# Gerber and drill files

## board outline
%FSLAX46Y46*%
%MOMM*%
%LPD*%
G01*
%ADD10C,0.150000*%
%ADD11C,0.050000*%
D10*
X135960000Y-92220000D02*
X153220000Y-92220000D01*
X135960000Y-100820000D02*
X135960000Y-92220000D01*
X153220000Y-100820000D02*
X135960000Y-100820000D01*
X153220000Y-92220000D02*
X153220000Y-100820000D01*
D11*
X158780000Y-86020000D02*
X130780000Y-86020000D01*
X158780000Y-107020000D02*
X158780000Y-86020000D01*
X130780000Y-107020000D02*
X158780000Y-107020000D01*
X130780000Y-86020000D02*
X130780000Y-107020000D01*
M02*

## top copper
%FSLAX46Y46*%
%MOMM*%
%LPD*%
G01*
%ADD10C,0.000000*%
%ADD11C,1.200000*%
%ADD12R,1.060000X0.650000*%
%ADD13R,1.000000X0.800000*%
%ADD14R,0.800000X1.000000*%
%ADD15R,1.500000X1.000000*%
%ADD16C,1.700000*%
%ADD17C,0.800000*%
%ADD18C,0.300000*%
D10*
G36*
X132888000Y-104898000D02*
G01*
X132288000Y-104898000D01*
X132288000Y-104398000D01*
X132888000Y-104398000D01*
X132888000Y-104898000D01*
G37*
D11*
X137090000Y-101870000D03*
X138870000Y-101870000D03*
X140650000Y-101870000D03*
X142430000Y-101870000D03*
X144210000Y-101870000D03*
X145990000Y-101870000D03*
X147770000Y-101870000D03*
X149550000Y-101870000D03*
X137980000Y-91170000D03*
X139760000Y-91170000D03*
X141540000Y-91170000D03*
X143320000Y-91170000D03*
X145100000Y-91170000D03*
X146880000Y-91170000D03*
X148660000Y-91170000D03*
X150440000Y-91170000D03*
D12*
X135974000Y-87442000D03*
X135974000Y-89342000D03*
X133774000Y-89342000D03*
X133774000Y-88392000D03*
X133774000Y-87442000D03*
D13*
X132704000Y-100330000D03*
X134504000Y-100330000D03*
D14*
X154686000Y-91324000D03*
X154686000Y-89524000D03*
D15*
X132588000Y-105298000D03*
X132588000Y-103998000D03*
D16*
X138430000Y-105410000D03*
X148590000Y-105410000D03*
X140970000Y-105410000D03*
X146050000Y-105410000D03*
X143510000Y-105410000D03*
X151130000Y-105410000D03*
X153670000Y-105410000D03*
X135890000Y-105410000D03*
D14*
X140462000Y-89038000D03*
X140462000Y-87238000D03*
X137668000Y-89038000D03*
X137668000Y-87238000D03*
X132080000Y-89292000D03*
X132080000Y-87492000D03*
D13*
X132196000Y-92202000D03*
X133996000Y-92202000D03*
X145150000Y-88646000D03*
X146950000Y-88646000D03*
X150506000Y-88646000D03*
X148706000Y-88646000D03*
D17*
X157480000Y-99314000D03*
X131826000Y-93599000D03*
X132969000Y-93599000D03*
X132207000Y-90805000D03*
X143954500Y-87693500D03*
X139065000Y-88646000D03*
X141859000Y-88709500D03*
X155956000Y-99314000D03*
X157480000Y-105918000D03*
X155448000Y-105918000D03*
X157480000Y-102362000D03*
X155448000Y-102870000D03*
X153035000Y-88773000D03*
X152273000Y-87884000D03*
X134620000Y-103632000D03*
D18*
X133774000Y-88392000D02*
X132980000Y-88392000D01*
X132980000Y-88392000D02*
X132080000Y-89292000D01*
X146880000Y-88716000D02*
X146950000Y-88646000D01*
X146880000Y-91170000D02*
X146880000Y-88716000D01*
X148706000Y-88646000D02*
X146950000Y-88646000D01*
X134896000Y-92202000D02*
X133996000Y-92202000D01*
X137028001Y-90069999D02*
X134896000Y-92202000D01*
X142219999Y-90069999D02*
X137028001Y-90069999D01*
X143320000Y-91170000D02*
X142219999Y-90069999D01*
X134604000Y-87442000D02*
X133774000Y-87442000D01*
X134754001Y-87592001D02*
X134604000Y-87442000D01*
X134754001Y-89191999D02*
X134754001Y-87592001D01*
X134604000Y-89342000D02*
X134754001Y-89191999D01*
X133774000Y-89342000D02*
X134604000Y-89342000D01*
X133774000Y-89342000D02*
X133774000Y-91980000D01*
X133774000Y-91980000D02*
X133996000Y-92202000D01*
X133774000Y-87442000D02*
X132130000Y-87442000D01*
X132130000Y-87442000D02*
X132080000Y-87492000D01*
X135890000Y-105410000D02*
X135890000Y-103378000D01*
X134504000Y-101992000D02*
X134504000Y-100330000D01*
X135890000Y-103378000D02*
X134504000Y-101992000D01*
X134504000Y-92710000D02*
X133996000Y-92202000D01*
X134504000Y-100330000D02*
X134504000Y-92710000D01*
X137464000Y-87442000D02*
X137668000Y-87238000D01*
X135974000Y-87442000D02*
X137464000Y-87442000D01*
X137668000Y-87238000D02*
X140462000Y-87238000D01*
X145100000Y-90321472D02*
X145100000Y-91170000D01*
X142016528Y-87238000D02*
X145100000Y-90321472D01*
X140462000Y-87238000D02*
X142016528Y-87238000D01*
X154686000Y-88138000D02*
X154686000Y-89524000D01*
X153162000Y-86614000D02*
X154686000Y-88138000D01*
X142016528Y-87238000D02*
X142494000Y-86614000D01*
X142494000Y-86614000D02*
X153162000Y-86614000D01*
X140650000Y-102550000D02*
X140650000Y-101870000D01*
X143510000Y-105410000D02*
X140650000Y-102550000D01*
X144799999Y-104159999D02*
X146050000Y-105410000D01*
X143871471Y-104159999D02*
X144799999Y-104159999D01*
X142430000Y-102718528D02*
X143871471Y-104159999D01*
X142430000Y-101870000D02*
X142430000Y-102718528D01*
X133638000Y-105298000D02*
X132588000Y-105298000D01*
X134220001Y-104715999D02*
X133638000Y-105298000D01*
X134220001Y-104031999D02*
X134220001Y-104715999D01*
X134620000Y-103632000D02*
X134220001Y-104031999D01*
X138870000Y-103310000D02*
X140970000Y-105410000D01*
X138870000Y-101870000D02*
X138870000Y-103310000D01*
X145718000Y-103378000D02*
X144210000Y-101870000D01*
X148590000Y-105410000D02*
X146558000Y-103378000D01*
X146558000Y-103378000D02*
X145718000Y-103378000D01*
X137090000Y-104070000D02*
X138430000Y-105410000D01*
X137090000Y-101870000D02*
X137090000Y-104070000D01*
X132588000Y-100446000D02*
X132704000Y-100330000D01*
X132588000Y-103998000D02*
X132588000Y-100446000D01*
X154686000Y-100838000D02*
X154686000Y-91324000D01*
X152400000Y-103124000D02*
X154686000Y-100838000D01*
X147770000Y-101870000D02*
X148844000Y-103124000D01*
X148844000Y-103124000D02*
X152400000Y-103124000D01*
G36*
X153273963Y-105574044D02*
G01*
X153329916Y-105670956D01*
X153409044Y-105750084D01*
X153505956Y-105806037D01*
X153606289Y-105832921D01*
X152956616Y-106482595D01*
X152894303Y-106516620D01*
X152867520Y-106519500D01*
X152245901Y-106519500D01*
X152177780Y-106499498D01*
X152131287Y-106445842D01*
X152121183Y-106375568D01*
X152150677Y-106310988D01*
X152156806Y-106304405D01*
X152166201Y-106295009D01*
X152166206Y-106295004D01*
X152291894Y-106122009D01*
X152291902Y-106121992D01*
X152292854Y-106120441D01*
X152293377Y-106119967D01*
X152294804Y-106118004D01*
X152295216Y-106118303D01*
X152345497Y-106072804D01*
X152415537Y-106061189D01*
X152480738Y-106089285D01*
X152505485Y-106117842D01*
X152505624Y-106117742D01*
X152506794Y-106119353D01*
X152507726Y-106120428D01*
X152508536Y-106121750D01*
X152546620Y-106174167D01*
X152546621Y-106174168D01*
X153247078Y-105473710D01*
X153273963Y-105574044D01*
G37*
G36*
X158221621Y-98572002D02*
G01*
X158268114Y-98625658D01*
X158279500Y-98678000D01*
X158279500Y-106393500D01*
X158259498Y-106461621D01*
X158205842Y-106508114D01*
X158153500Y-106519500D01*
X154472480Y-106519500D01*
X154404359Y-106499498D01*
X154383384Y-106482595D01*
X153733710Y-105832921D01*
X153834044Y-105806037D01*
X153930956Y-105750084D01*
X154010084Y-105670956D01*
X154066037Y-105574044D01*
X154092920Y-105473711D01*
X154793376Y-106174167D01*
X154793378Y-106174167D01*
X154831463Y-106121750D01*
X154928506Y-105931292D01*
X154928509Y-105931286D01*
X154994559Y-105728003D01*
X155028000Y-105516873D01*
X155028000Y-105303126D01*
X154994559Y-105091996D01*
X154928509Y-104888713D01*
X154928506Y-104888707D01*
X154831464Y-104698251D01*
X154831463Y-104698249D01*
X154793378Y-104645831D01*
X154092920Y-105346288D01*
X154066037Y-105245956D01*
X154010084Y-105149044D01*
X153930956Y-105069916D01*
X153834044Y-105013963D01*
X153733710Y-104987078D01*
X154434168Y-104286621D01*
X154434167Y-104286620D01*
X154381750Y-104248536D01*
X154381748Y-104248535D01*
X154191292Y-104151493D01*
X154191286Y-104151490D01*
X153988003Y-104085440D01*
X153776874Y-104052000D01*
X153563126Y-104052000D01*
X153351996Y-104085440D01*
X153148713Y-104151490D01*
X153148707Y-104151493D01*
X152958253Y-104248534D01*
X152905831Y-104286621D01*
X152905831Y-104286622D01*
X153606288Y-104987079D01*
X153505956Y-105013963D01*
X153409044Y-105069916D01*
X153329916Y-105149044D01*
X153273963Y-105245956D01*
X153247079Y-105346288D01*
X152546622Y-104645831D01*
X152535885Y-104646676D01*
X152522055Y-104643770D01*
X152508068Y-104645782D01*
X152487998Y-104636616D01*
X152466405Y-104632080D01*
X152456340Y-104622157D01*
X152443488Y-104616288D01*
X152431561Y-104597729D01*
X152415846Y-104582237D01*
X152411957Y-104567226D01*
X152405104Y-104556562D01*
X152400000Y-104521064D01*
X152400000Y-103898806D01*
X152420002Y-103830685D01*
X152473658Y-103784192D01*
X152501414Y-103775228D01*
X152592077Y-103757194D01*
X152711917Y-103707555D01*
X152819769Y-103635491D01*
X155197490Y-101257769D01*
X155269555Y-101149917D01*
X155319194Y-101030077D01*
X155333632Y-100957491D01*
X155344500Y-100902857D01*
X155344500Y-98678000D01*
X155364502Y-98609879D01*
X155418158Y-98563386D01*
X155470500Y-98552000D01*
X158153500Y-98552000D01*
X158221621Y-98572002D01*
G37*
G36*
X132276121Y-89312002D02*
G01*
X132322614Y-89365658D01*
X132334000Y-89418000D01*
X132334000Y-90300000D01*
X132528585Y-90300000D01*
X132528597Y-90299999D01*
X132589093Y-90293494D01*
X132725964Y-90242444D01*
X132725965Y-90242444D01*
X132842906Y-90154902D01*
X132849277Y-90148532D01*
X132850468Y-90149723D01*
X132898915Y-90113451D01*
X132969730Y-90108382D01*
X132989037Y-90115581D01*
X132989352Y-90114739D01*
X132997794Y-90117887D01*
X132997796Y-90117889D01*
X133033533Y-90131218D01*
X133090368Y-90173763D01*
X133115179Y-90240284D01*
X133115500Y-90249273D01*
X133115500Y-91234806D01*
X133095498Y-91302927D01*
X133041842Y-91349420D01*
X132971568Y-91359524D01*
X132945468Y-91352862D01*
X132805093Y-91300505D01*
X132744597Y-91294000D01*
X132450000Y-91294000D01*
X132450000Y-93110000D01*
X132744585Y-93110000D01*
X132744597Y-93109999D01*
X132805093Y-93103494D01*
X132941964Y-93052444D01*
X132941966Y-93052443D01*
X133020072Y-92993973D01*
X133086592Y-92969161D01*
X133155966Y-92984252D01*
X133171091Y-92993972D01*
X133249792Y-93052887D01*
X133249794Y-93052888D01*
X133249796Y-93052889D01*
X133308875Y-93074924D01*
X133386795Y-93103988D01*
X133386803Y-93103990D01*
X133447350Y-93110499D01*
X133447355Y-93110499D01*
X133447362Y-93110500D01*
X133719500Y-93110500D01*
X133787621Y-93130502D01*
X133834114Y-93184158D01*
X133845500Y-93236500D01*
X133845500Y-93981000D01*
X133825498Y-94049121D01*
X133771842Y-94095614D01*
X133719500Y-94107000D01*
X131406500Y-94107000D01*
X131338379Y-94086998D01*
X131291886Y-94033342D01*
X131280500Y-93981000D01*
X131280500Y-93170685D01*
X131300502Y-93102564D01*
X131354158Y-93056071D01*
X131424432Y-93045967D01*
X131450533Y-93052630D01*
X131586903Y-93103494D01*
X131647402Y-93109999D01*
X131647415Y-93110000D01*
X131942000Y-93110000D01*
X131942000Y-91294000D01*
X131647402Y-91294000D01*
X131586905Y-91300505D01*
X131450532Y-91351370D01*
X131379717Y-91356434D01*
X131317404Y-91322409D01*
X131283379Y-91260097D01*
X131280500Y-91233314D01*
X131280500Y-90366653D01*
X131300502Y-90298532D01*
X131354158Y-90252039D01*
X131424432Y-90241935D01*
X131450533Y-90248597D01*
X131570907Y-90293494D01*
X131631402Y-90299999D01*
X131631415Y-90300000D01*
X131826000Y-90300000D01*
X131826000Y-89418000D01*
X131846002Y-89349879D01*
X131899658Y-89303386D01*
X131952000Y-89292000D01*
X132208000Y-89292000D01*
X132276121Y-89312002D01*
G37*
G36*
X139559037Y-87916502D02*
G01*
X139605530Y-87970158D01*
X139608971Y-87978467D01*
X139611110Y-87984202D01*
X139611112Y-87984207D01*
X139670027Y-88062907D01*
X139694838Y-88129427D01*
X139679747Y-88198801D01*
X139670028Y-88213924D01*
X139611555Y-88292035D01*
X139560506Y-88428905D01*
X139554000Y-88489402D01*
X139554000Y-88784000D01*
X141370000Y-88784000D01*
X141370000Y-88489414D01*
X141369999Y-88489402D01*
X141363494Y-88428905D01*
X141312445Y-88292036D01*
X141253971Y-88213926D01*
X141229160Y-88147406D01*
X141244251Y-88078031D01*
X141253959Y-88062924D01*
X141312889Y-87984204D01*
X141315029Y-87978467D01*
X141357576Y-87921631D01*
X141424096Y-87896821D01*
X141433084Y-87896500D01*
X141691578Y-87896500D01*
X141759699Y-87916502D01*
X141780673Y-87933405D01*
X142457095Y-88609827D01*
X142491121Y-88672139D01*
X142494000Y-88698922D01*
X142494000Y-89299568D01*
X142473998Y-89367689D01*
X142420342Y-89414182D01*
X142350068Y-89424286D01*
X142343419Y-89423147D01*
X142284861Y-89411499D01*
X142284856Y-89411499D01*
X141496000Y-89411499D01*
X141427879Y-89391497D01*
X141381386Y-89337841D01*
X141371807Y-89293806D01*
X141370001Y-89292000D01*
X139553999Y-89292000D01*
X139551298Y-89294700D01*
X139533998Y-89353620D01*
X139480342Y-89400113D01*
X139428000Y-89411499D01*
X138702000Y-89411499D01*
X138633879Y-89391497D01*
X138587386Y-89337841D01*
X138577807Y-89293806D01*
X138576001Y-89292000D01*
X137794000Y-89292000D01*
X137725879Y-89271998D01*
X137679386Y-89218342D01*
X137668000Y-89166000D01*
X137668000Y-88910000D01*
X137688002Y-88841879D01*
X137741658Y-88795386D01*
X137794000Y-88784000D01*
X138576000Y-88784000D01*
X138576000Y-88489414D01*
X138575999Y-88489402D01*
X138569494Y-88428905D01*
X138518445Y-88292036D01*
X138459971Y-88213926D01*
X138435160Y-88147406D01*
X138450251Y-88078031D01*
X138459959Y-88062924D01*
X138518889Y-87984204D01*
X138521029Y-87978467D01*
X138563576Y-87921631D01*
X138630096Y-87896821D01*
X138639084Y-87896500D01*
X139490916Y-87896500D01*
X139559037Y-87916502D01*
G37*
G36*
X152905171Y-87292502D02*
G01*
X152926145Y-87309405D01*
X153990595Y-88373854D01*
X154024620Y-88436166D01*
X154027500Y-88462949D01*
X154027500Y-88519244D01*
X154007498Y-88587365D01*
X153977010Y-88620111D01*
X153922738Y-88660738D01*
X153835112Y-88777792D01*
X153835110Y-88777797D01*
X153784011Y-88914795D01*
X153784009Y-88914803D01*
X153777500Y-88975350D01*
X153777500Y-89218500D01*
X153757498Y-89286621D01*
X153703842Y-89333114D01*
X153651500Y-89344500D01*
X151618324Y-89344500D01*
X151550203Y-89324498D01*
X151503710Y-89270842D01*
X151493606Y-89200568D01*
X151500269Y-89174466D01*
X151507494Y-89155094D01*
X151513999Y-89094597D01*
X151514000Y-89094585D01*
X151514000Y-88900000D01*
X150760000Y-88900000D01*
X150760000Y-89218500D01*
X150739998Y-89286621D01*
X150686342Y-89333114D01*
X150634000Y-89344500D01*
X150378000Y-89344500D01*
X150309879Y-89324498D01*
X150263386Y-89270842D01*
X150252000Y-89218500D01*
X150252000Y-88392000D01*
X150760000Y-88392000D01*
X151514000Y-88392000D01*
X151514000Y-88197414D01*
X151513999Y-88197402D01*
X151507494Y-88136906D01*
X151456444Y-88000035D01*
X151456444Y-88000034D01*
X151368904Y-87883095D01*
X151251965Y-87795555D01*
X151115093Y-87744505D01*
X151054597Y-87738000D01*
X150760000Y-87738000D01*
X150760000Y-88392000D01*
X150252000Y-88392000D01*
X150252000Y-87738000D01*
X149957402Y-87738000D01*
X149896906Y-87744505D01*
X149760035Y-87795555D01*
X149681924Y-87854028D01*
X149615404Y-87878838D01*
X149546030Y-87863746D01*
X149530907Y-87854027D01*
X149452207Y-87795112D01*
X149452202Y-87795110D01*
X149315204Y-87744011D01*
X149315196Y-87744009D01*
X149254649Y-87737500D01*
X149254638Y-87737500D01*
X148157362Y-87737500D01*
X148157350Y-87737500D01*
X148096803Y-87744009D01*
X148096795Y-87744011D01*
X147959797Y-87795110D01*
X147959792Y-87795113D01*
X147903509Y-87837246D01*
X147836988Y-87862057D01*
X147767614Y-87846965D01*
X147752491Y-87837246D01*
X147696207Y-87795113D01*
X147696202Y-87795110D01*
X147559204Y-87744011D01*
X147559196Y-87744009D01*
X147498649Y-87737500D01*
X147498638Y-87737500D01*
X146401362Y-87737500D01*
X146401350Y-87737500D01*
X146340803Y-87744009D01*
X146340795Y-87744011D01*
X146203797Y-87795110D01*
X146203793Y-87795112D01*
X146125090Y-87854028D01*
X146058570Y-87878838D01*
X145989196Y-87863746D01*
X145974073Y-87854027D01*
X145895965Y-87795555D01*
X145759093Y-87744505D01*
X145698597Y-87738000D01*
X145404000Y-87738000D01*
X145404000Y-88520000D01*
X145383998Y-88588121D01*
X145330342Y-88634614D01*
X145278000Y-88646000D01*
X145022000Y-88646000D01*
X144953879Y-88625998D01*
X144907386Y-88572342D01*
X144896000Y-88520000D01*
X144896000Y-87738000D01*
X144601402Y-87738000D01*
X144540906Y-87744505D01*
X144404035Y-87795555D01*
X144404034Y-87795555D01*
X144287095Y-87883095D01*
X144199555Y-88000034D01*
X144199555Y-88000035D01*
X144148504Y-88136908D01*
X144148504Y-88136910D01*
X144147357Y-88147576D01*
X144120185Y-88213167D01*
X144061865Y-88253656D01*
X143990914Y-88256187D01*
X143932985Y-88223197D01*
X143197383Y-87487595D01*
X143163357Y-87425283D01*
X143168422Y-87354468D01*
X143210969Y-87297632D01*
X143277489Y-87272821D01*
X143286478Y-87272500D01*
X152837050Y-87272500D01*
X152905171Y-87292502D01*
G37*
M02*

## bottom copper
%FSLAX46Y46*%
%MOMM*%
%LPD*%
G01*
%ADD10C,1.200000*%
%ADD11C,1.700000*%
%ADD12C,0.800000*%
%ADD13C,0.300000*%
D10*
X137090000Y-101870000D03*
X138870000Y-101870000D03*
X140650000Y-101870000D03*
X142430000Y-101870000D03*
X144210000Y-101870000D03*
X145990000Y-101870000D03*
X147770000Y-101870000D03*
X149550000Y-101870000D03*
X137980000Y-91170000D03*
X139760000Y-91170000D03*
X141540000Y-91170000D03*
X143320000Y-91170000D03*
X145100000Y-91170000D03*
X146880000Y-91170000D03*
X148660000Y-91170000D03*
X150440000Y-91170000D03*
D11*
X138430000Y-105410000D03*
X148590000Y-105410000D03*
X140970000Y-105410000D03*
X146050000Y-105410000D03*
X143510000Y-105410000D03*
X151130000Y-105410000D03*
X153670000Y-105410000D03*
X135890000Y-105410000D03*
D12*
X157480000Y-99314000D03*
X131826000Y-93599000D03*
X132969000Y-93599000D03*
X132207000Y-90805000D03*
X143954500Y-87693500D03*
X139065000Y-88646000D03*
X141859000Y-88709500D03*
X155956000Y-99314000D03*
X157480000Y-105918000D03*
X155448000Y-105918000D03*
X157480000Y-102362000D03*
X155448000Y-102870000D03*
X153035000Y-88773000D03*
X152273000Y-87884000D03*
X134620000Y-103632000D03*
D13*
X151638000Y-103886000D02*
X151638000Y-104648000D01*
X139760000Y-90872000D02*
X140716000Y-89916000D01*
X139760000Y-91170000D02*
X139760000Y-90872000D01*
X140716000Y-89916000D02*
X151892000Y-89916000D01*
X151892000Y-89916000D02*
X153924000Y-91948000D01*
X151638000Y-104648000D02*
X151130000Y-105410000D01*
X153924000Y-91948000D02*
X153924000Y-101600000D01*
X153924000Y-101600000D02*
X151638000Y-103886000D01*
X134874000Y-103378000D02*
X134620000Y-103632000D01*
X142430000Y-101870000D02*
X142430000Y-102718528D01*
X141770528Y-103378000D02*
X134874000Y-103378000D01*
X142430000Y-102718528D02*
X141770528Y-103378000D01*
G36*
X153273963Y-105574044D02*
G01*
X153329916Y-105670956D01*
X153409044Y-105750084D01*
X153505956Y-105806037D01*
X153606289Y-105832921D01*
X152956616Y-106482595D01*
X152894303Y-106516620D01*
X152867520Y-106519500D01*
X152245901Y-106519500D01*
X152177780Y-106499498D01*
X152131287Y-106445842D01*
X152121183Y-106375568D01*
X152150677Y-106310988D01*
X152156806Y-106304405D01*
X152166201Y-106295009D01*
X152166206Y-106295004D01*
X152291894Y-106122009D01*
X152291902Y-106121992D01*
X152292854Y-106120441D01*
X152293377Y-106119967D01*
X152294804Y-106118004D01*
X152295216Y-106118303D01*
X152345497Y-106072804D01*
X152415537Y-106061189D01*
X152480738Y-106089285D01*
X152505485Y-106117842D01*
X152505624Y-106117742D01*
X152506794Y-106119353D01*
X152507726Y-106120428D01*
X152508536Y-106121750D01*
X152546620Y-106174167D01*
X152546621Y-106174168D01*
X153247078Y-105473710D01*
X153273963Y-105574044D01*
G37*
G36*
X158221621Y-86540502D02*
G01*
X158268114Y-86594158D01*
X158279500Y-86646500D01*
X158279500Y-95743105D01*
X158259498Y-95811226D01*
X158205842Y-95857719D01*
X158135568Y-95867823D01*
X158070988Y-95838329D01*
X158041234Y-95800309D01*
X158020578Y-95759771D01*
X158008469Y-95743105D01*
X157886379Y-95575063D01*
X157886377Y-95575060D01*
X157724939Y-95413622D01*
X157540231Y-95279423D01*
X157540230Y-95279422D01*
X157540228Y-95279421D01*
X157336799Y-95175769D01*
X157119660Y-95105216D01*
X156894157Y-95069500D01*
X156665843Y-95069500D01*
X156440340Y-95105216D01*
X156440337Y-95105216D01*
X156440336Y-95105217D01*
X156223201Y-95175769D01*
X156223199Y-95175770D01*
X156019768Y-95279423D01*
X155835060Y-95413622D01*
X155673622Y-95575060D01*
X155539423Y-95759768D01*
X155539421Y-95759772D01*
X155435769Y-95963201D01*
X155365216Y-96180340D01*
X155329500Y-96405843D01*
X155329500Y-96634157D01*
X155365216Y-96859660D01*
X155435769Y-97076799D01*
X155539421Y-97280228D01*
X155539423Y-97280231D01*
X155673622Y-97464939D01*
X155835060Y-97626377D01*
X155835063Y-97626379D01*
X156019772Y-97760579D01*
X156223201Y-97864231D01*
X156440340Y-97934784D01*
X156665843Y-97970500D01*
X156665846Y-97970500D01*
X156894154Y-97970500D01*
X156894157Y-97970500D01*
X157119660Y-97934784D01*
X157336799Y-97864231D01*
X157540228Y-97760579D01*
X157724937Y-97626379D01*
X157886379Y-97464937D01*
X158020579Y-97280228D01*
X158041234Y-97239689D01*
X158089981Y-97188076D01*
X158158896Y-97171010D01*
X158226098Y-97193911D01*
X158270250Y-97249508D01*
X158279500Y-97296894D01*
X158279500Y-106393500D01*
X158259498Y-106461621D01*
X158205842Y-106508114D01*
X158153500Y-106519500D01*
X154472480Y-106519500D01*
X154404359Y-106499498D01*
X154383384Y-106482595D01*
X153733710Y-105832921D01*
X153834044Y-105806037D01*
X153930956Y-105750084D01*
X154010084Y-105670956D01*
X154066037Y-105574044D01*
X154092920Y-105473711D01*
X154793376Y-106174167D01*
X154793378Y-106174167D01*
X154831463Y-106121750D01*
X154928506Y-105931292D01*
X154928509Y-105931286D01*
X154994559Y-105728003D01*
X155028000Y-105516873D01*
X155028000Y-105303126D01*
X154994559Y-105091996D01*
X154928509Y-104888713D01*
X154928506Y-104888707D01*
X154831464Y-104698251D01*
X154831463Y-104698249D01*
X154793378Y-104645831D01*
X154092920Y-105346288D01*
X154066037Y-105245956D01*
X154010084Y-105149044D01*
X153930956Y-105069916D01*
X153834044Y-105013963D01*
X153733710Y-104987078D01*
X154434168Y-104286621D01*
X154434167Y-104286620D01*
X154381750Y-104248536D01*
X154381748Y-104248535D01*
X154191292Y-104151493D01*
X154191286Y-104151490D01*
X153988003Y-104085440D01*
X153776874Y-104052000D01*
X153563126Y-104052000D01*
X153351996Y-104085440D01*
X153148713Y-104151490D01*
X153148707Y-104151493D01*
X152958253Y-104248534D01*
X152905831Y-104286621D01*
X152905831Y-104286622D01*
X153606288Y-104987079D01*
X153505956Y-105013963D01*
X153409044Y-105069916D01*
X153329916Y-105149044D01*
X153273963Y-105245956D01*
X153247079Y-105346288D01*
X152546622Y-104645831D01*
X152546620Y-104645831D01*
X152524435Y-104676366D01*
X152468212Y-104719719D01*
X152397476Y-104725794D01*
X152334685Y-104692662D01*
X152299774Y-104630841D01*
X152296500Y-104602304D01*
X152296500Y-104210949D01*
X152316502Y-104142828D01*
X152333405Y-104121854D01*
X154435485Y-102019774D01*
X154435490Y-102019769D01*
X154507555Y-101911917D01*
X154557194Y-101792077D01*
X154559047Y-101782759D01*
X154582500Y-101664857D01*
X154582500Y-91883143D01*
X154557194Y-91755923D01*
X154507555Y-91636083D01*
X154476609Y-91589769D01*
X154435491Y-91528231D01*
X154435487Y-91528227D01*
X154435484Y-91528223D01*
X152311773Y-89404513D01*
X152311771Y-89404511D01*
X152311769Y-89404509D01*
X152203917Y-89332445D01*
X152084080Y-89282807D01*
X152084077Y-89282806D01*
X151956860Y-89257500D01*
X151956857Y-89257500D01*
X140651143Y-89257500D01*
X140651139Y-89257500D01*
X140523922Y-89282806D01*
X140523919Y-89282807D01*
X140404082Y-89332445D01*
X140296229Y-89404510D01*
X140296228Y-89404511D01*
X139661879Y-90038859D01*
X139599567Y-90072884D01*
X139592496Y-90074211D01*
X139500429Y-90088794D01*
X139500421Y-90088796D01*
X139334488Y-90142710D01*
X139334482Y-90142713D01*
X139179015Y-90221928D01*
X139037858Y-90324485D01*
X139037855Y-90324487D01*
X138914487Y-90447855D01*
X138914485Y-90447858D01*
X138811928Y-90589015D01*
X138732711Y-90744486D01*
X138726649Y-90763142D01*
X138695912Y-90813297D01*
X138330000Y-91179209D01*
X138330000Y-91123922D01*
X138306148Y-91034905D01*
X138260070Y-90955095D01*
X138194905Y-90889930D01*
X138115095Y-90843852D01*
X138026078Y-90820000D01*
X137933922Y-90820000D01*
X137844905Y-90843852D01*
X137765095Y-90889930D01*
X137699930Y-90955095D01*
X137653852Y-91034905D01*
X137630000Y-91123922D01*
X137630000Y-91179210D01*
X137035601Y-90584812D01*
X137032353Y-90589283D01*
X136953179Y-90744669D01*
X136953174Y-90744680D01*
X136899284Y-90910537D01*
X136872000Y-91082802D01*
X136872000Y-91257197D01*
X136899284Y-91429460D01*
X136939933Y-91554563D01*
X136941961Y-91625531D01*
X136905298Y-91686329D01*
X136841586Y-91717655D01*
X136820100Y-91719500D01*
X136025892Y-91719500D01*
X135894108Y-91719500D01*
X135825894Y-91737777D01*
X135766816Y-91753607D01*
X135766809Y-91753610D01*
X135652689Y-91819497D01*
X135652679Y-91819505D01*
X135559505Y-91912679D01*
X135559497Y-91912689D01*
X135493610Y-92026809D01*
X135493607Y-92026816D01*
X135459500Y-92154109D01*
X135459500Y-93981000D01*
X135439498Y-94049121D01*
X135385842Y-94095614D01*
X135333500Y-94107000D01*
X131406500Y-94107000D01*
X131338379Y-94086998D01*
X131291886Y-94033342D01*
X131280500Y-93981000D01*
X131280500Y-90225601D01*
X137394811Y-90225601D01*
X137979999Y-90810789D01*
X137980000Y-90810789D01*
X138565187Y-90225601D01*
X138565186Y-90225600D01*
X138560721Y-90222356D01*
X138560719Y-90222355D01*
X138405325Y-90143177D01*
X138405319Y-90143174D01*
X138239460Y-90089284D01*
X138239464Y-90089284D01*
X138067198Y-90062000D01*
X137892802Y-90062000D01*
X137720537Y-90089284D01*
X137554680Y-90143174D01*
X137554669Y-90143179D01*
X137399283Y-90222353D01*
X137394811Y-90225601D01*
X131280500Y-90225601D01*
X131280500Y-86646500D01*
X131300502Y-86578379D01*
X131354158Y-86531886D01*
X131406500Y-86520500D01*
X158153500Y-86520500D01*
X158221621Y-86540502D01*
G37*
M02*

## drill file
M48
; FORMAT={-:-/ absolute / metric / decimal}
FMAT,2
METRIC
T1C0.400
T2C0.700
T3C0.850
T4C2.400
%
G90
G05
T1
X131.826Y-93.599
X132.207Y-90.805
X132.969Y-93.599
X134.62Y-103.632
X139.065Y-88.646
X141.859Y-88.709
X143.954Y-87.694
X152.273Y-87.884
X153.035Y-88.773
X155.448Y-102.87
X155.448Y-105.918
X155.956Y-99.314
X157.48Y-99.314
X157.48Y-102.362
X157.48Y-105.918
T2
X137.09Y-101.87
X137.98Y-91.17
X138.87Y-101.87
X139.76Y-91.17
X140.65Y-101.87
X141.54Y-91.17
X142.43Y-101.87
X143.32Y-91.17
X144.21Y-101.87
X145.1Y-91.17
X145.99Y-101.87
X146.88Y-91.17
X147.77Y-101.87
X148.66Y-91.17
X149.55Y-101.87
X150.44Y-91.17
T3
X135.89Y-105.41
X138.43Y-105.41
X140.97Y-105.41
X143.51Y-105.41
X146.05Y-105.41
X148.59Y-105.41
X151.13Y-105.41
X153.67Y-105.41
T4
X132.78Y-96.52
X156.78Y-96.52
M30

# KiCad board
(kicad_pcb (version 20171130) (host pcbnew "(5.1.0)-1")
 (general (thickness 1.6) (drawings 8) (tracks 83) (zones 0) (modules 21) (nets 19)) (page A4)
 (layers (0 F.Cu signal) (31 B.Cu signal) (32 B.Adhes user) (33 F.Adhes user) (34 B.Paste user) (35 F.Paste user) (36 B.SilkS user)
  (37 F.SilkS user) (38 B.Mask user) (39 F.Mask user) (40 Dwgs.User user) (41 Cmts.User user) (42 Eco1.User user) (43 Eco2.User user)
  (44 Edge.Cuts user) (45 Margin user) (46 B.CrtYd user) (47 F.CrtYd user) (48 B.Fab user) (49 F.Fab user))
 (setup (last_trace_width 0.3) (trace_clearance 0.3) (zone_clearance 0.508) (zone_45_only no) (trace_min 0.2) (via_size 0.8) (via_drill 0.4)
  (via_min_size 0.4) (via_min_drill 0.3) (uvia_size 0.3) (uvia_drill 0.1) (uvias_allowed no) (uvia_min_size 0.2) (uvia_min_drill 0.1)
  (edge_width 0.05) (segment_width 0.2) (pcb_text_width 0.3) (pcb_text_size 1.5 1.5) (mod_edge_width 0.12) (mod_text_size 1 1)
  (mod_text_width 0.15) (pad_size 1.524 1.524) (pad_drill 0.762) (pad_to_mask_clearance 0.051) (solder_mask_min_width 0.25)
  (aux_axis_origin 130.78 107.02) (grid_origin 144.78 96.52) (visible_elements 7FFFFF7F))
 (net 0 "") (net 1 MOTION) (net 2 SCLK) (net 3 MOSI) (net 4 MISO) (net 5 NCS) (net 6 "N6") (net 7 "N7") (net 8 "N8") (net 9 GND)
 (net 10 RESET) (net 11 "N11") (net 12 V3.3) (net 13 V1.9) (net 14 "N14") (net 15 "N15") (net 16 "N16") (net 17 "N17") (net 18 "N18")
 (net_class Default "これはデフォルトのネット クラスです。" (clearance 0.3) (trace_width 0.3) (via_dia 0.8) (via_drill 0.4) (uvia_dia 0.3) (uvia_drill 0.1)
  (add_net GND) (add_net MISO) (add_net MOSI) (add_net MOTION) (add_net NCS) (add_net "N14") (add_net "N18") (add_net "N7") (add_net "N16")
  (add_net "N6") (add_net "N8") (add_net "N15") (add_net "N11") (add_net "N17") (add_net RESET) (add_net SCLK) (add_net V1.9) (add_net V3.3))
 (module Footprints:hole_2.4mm (layer F.Cu) (at 132.78 96.52)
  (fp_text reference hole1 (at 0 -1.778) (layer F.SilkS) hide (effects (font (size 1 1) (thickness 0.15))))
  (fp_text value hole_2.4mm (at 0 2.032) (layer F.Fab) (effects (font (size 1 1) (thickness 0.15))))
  (pad "" np_thru_hole circle (at 0 0) (size 2.4 2.4) (drill 2.4) (layers *.Cu *.Mask)))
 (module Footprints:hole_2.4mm (layer F.Cu) (at 156.78 96.52)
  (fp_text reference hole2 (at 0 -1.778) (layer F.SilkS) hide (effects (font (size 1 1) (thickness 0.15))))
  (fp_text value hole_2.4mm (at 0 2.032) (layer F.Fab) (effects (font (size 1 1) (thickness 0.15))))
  (pad "" np_thru_hole circle (at 0 0) (size 2.4 2.4) (drill 2.4) (layers *.Cu *.Mask)))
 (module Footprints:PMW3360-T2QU (layer F.Cu) (at 144.78 96.52)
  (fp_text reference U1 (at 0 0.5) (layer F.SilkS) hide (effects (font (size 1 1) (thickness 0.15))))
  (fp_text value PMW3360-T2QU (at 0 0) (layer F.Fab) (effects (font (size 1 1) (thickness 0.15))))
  (pad 9 thru_hole circle (at -7.69 5.35) (size 1.2 1.2) (drill 0.7) (layers *.Cu *.Mask) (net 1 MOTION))
  (pad 10 thru_hole circle (at -5.91 5.35) (size 1.2 1.2) (drill 0.7) (layers *.Cu *.Mask) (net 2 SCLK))
  (pad 11 thru_hole circle (at -4.13 5.35) (size 1.2 1.2) (drill 0.7) (layers *.Cu *.Mask) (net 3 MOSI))
  (pad 12 thru_hole circle (at -2.35 5.35) (size 1.2 1.2) (drill 0.7) (layers *.Cu *.Mask) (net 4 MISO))
  (pad 13 thru_hole circle (at -0.57 5.35) (size 1.2 1.2) (drill 0.7) (layers *.Cu *.Mask) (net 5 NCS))
  (pad 14 thru_hole circle (at 1.21 5.35) (size 1.2 1.2) (drill 0.7) (layers *.Cu *.Mask) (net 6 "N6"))
  (pad 15 thru_hole circle (at 2.99 5.35) (size 1.2 1.2) (drill 0.7) (layers *.Cu *.Mask) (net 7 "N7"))
  (pad 16 thru_hole circle (at 4.77 5.35) (size 1.2 1.2) (drill 0.7) (layers *.Cu *.Mask) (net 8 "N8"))
  (pad 8 thru_hole circle (at -6.8 -5.35) (size 1.2 1.2) (drill 0.7) (layers *.Cu *.Mask) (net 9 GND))
  (pad 7 thru_hole circle (at -5.02 -5.35) (size 1.2 1.2) (drill 0.7) (layers *.Cu *.Mask) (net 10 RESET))
  (pad 6 thru_hole circle (at -3.24 -5.35) (size 1.2 1.2) (drill 0.7) (layers *.Cu *.Mask) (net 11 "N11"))
  (pad 5 thru_hole circle (at -1.46 -5.35) (size 1.2 1.2) (drill 0.7) (layers *.Cu *.Mask) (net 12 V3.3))
  (pad 4 thru_hole circle (at 0.32 -5.35) (size 1.2 1.2) (drill 0.7) (layers *.Cu *.Mask) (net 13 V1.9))
  (pad 3 thru_hole circle (at 2.1 -5.35) (size 1.2 1.2) (drill 0.7) (layers *.Cu *.Mask) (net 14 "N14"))
  (pad 2 thru_hole circle (at 3.88 -5.35) (size 1.2 1.2) (drill 0.7) (layers *.Cu *.Mask) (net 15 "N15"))
  (pad 1 thru_hole circle (at 5.66 -5.35) (size 1.2 1.2) (drill 0.7) (layers *.Cu *.Mask) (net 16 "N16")))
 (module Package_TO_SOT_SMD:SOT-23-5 (layer F.Cu) (at 134.874 88.392)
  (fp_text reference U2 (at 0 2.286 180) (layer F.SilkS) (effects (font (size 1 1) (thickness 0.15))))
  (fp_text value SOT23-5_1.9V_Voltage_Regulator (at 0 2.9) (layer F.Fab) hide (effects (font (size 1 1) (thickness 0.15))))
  (pad 5 smd rect (at 1.1 -0.95) (size 1.06 0.65) (layers F.Cu F.Paste F.Mask) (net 13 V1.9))
  (pad 4 smd rect (at 1.1 0.95) (size 1.06 0.65) (layers F.Cu F.Paste F.Mask) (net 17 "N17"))
  (pad 3 smd rect (at -1.1 0.95) (size 1.06 0.65) (layers F.Cu F.Paste F.Mask) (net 12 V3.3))
  (pad 2 smd rect (at -1.1 0) (size 1.06 0.65) (layers F.Cu F.Paste F.Mask) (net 9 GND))
  (pad 1 smd rect (at -1.1 -0.95) (size 1.06 0.65) (layers F.Cu F.Paste F.Mask) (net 12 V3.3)))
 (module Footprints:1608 (layer F.Cu) (at 133.604 100.33 180)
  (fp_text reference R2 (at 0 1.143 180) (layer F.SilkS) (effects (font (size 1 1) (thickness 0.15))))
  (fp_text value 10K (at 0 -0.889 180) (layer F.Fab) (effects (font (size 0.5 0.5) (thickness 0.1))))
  (pad 2 smd rect (at 0.9 0 180) (size 1 0.8) (layers F.Cu F.Paste F.Mask) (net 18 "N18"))
  (pad 1 smd rect (at -0.9 0 180) (size 1 0.8) (layers F.Cu F.Paste F.Mask) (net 12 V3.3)))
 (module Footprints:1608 (layer F.Cu) (at 154.686 90.424 270)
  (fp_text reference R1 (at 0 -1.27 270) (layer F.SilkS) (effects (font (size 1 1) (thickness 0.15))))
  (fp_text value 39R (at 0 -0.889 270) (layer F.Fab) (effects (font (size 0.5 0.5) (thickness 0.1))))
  (pad 2 smd rect (at 0.9 0 270) (size 1 0.8) (layers F.Cu F.Paste F.Mask) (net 7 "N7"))
  (pad 1 smd rect (at -0.9 0 270) (size 1 0.8) (layers F.Cu F.Paste F.Mask) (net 13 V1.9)))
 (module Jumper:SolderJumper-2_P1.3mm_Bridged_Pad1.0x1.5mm (layer F.Cu) (at 132.588 104.648 270)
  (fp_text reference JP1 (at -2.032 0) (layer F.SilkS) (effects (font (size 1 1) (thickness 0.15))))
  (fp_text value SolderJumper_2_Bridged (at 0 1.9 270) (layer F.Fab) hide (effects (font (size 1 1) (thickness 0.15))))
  (fp_poly (pts (xy -0.25 -0.3) (xy 0.25 -0.3) (xy 0.25 0.3) (xy -0.25 0.3)) (layer F.Cu) (width 0))
  (pad 2 smd rect (at 0.65 0 270) (size 1 1.5) (layers F.Cu F.Mask) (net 4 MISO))
  (pad 1 smd rect (at -0.65 0 270) (size 1 1.5) (layers F.Cu F.Mask) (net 18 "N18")))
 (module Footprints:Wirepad (layer F.Cu) (at 138.43 105.41 180)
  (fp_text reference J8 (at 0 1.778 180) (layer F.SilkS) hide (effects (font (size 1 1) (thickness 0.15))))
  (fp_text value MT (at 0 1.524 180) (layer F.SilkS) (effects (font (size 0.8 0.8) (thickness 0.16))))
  (pad 1 thru_hole circle (at 0 0 180) (size 1.7 1.7) (drill 0.85) (layers *.Cu *.Mask) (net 1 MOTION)))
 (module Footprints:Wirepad (layer F.Cu) (at 148.59 105.41 180)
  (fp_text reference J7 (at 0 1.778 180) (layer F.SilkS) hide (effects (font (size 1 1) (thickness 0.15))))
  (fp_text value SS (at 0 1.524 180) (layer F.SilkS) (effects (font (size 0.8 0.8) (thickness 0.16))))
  (pad 1 thru_hole circle (at 0 0 180) (size 1.7 1.7) (drill 0.85) (layers *.Cu *.Mask) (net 5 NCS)))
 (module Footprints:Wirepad (layer F.Cu) (at 140.97 105.41 180)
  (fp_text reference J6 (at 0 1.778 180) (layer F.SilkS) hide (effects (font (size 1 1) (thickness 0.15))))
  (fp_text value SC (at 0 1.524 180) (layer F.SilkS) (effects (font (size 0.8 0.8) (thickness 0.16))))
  (pad 1 thru_hole circle (at 0 0 180) (size 1.7 1.7) (drill 0.85) (layers *.Cu *.Mask) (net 2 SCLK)))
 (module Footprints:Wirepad (layer F.Cu) (at 146.05 105.41 180)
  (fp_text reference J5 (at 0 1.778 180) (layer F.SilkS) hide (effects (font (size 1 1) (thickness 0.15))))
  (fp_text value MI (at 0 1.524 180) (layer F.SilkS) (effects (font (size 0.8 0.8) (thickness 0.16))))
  (pad 1 thru_hole circle (at 0 0 180) (size 1.7 1.7) (drill 0.85) (layers *.Cu *.Mask) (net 4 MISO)))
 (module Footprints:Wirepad (layer F.Cu) (at 143.51 105.41 180)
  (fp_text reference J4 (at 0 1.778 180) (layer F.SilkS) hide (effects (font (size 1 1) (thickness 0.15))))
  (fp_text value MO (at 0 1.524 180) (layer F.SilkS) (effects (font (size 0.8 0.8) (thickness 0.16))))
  (pad 1 thru_hole circle (at 0 0 180) (size 1.7 1.7) (drill 0.85) (layers *.Cu *.Mask) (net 3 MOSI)))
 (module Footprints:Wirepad (layer F.Cu) (at 151.13 105.41 180)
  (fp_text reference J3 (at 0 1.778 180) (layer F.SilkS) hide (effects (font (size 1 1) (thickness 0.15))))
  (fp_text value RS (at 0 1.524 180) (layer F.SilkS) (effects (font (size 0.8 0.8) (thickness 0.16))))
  (pad 1 thru_hole circle (at 0 0 180) (size 1.7 1.7) (drill 0.85) (layers *.Cu *.Mask) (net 10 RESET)))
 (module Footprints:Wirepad (layer F.Cu) (at 153.67 105.41 180)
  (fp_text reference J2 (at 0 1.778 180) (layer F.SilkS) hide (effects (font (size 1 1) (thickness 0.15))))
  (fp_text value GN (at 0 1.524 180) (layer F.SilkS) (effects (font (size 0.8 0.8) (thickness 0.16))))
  (pad 1 thru_hole circle (at 0 0 180) (size 1.7 1.7) (drill 0.85) (layers *.Cu *.Mask) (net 9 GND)))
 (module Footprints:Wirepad (layer F.Cu) (at 135.89 105.41 180)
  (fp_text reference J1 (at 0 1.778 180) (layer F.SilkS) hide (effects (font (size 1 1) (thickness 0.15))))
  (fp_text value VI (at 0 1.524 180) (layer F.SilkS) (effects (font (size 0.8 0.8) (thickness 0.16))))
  (pad 1 thru_hole circle (at 0 0 180) (size 1.7 1.7) (drill 0.85) (layers *.Cu *.Mask) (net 12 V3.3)))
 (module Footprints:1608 (layer F.Cu) (at 140.462 88.138 270)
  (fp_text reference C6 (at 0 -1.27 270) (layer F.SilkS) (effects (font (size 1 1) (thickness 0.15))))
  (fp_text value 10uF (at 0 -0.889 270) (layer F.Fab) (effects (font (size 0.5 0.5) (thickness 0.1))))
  (pad 2 smd rect (at 0.9 0 270) (size 1 0.8) (layers F.Cu F.Paste F.Mask) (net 9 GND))
  (pad 1 smd rect (at -0.9 0 270) (size 1 0.8) (layers F.Cu F.Paste F.Mask) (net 13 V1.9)))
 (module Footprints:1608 (layer F.Cu) (at 137.668 88.138 270)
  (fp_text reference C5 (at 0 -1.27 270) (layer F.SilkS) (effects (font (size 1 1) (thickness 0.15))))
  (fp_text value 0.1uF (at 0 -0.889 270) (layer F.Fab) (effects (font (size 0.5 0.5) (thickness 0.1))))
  (pad 2 smd rect (at 0.9 0 270) (size 1 0.8) (layers F.Cu F.Paste F.Mask) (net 9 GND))
  (pad 1 smd rect (at -0.9 0 270) (size 1 0.8) (layers F.Cu F.Paste F.Mask) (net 13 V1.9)))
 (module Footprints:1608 (layer F.Cu) (at 132.08 88.392 270)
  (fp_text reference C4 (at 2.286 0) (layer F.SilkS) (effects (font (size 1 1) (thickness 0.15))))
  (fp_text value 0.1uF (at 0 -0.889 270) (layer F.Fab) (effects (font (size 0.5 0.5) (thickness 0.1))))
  (pad 2 smd rect (at 0.9 0 270) (size 1 0.8) (layers F.Cu F.Paste F.Mask) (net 9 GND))
  (pad 1 smd rect (at -0.9 0 270) (size 1 0.8) (layers F.Cu F.Paste F.Mask) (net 12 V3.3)))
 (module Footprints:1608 (layer F.Cu) (at 133.096 92.202 180)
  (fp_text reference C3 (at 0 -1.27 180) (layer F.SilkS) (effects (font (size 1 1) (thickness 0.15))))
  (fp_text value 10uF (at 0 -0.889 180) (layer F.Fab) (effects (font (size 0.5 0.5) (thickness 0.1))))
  (pad 2 smd rect (at 0.9 0 180) (size 1 0.8) (layers F.Cu F.Paste F.Mask) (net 9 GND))
  (pad 1 smd rect (at -0.9 0 180) (size 1 0.8) (layers F.Cu F.Paste F.Mask) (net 12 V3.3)))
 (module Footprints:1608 (layer F.Cu) (at 146.05 88.646 180)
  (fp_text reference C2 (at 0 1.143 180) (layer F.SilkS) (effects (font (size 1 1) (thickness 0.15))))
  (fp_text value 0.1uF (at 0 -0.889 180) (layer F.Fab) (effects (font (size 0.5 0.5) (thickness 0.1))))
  (pad 2 smd rect (at 0.9 0 180) (size 1 0.8) (layers F.Cu F.Paste F.Mask) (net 9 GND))
  (pad 1 smd rect (at -0.9 0 180) (size 1 0.8) (layers F.Cu F.Paste F.Mask) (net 14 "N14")))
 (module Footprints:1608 (layer F.Cu) (at 149.606 88.646)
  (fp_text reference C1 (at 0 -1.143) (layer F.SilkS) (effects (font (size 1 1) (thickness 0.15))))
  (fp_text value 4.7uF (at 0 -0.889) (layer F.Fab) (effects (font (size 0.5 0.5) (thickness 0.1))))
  (pad 2 smd rect (at 0.9 0) (size 1 0.8) (layers F.Cu F.Paste F.Mask) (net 9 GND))
  (pad 1 smd rect (at -0.9 0) (size 1 0.8) (layers F.Cu F.Paste F.Mask) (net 14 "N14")))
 (gr_line (start 135.96 92.22) (end 153.22 92.22) (layer Edge.Cuts) (width 0.15))
 (gr_line (start 135.96 100.82) (end 135.96 92.22) (layer Edge.Cuts) (width 0.15))
 (gr_line (start 153.22 100.82) (end 135.96 100.82) (layer Edge.Cuts) (width 0.15))
 (gr_line (start 153.22 92.22) (end 153.22 100.82) (layer Edge.Cuts) (width 0.15))
 (gr_line (start 158.78 86.02) (end 130.78 86.02) (layer Edge.Cuts) (width 0.05))
 (gr_line (start 158.78 107.02) (end 158.78 86.02) (layer Edge.Cuts) (width 0.05))
 (gr_line (start 130.78 107.02) (end 158.78 107.02) (layer Edge.Cuts) (width 0.05))
 (gr_line (start 130.78 86.02) (end 130.78 107.02) (layer Edge.Cuts) (width 0.05))
 (segment (start 133.774 88.392) (end 132.98 88.392) (width 0.3) (layer F.Cu) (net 9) (status 10))
 (segment (start 132.98 88.392) (end 132.08 89.292) (width 0.3) (layer F.Cu) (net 9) (status 20))
 (via (at 157.48 99.314) (size 0.8) (drill 0.4) (layers F.Cu B.Cu) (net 9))
 (via (at 131.826 93.599) (size 0.8) (drill 0.4) (layers F.Cu B.Cu) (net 9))
 (via (at 132.969 93.599) (size 0.8) (drill 0.4) (layers F.Cu B.Cu) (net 9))
 (via (at 132.207 90.805) (size 0.8) (drill 0.4) (layers F.Cu B.Cu) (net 9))
 (via (at 143.9545 87.6935) (size 0.8) (drill 0.4) (layers F.Cu B.Cu) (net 9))
 (via (at 139.065 88.646) (size 0.8) (drill 0.4) (layers F.Cu B.Cu) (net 9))
 (via (at 141.859 88.7095) (size 0.8) (drill 0.4) (layers F.Cu B.Cu) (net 9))
 (via (at 155.956 99.314) (size 0.8) (drill 0.4) (layers F.Cu B.Cu) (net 9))
 (via (at 157.48 105.918) (size 0.8) (drill 0.4) (layers F.Cu B.Cu) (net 9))
 (via (at 155.448 105.918) (size 0.8) (drill 0.4) (layers F.Cu B.Cu) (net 9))
 (via (at 157.48 102.362) (size 0.8) (drill 0.4) (layers F.Cu B.Cu) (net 9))
 (via (at 155.448 102.87) (size 0.8) (drill 0.4) (layers F.Cu B.Cu) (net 9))
 (via (at 153.035 88.773) (size 0.8) (drill 0.4) (layers F.Cu B.Cu) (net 9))
 (via (at 152.273 87.884) (size 0.8) (drill 0.4) (layers F.Cu B.Cu) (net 9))
 (segment (start 146.88 88.716) (end 146.95 88.646) (width 0.3) (layer F.Cu) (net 14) (status 30))
 (segment (start 146.88 91.17) (end 146.88 88.716) (width 0.3) (layer F.Cu) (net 14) (status 30))
 (segment (start 148.706 88.646) (end 146.95 88.646) (width 0.3) (layer F.Cu) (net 14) (status 30))
 (segment (start 134.896 92.202) (end 133.996 92.202) (width 0.3) (layer F.Cu) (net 12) (status 20))
 (segment (start 137.028001 90.069999) (end 134.896 92.202) (width 0.3) (layer F.Cu) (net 12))
 (segment (start 142.219999 90.069999) (end 137.028001 90.069999) (width 0.3) (layer F.Cu) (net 12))
 (segment (start 143.32 91.17) (end 142.219999 90.069999) (width 0.3) (layer F.Cu) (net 12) (status 10))
 (segment (start 134.604 87.442) (end 133.774 87.442) (width 0.3) (layer F.Cu) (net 12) (status 20))
 (segment (start 134.754001 87.592001) (end 134.604 87.442) (width 0.3) (layer F.Cu) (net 12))
 (segment (start 134.754001 89.191999) (end 134.754001 87.592001) (width 0.3) (layer F.Cu) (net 12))
 (segment (start 134.604 89.342) (end 134.754001 89.191999) (width 0.3) (layer F.Cu) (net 12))
 (segment (start 133.774 89.342) (end 134.604 89.342) (width 0.3) (layer F.Cu) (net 12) (status 10))
 (segment (start 133.774 89.342) (end 133.774 91.98) (width 0.3) (layer F.Cu) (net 12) (status 30))
 (segment (start 133.774 91.98) (end 133.996 92.202) (width 0.3) (layer F.Cu) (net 12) (status 30))
 (segment (start 133.774 87.442) (end 132.13 87.442) (width 0.3) (layer F.Cu) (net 12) (status 30))
 (segment (start 132.13 87.442) (end 132.08 87.492) (width 0.3) (layer F.Cu) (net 12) (status 30))
 (segment (start 135.89 105.41) (end 135.89 103.378) (width 0.3) (layer F.Cu) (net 12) (status 10))
 (segment (start 134.504 101.992) (end 134.504 100.33) (width 0.3) (layer F.Cu) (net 12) (status 20))
 (segment (start 135.89 103.378) (end 134.504 101.992) (width 0.3) (layer F.Cu) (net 12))
 (segment (start 134.504 92.71) (end 133.996 92.202) (width 0.3) (layer F.Cu) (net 12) (status 20))
 (segment (start 134.504 100.33) (end 134.504 92.71) (width 0.3) (layer F.Cu) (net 12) (status 10))
 (segment (start 137.464 87.442) (end 137.668 87.238) (width 0.3) (layer F.Cu) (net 13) (status 30))
 (segment (start 135.974 87.442) (end 137.464 87.442) (width 0.3) (layer F.Cu) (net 13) (status 30))
 (segment (start 137.668 87.238) (end 140.462 87.238) (width 0.3) (layer F.Cu) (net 13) (status 30))
 (segment (start 145.1 90.321472) (end 145.1 91.17) (width 0.3) (layer F.Cu) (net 13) (status 20))
 (segment (start 142.016528 87.238) (end 145.1 90.321472) (width 0.3) (layer F.Cu) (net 13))
 (segment (start 140.462 87.238) (end 142.016528 87.238) (width 0.3) (layer F.Cu) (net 13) (status 10))
 (segment (start 154.686 88.138) (end 154.686 89.524) (width 0.3) (layer F.Cu) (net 13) (status 20))
 (segment (start 153.162 86.614) (end 154.686 88.138) (width 0.3) (layer F.Cu) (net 13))
 (segment (start 142.016528 87.238) (end 142.494 86.614) (width 0.3) (layer F.Cu) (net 13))
 (segment (start 142.494 86.614) (end 153.162 86.614) (width 0.3) (layer F.Cu) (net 13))
 (segment (start 151.638 103.886) (end 151.638 104.648) (width 0.3) (layer B.Cu) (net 10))
 (segment (start 139.76 90.872) (end 140.716 89.916) (width 0.3) (layer B.Cu) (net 10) (status 10))
 (segment (start 139.76 91.17) (end 139.76 90.872) (width 0.3) (layer B.Cu) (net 10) (status 30))
 (segment (start 140.716 89.916) (end 151.892 89.916) (width 0.3) (layer B.Cu) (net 10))
 (segment (start 151.892 89.916) (end 153.924 91.948) (width 0.3) (layer B.Cu) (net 10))
 (segment (start 151.638 104.648) (end 151.13 105.41) (width 0.3) (layer B.Cu) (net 10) (status 20))
 (segment (start 153.924 91.948) (end 153.924 101.6) (width 0.3) (layer B.Cu) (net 10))
 (segment (start 153.924 101.6) (end 151.638 103.886) (width 0.3) (layer B.Cu) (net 10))
 (segment (start 140.65 102.55) (end 140.65 101.87) (width 0.3) (layer F.Cu) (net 3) (status 20))
 (segment (start 143.51 105.41) (end 140.65 102.55) (width 0.3) (layer F.Cu) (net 3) (status 10))
 (segment (start 144.799999 104.159999) (end 146.05 105.41) (width 0.3) (layer F.Cu) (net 4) (status 20))
 (segment (start 143.871471 104.159999) (end 144.799999 104.159999) (width 0.3) (layer F.Cu) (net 4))
 (segment (start 142.43 102.718528) (end 143.871471 104.159999) (width 0.3) (layer F.Cu) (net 4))
 (segment (start 142.43 101.87) (end 142.43 102.718528) (width 0.3) (layer F.Cu) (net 4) (status 10))
 (segment (start 134.874 103.378) (end 134.62 103.632) (width 0.3) (layer B.Cu) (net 4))
 (segment (start 142.43 101.87) (end 142.43 102.718528) (width 0.3) (layer B.Cu) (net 4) (status 10))
 (segment (start 141.770528 103.378) (end 134.874 103.378) (width 0.3) (layer B.Cu) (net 4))
 (segment (start 142.43 102.718528) (end 141.770528 103.378) (width 0.3) (layer B.Cu) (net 4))
 (via (at 134.62 103.632) (size 0.8) (drill 0.4) (layers F.Cu B.Cu) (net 4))
 (segment (start 133.638 105.298) (end 132.588 105.298) (width 0.3) (layer F.Cu) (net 4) (status 20))
 (segment (start 134.220001 104.715999) (end 133.638 105.298) (width 0.3) (layer F.Cu) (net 4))
 (segment (start 134.220001 104.031999) (end 134.220001 104.715999) (width 0.3) (layer F.Cu) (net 4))
 (segment (start 134.62 103.632) (end 134.220001 104.031999) (width 0.3) (layer F.Cu) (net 4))
 (segment (start 138.87 103.31) (end 140.97 105.41) (width 0.3) (layer F.Cu) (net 2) (status 20))
 (segment (start 138.87 101.87) (end 138.87 103.31) (width 0.3) (layer F.Cu) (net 2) (status 10))
 (segment (start 145.718 103.378) (end 144.21 101.87) (width 0.3) (layer F.Cu) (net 5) (status 20))
 (segment (start 148.59 105.41) (end 146.558 103.378) (width 0.3) (layer F.Cu) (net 5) (status 10))
 (segment (start 146.558 103.378) (end 145.718 103.378) (width 0.3) (layer F.Cu) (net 5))
 (segment (start 137.09 104.07) (end 138.43 105.41) (width 0.3) (layer F.Cu) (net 1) (status 20))
 (segment (start 137.09 101.87) (end 137.09 104.07) (width 0.3) (layer F.Cu) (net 1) (status 10))
 (segment (start 132.588 100.446) (end 132.704 100.33) (width 0.3) (layer F.Cu) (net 18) (status 30))
 (segment (start 132.588 103.998) (end 132.588 100.446) (width 0.3) (layer F.Cu) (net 18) (status 30))
 (segment (start 154.686 100.838) (end 154.686 91.324) (width 0.3) (layer F.Cu) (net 7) (status 20))
 (segment (start 152.4 103.124) (end 154.686 100.838) (width 0.3) (layer F.Cu) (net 7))
 (segment (start 147.77 101.87) (end 148.844 103.124) (width 0.3) (layer F.Cu) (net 7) (status 10))
 (segment (start 148.844 103.124) (end 152.4 103.124) (width 0.3) (layer F.Cu) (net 7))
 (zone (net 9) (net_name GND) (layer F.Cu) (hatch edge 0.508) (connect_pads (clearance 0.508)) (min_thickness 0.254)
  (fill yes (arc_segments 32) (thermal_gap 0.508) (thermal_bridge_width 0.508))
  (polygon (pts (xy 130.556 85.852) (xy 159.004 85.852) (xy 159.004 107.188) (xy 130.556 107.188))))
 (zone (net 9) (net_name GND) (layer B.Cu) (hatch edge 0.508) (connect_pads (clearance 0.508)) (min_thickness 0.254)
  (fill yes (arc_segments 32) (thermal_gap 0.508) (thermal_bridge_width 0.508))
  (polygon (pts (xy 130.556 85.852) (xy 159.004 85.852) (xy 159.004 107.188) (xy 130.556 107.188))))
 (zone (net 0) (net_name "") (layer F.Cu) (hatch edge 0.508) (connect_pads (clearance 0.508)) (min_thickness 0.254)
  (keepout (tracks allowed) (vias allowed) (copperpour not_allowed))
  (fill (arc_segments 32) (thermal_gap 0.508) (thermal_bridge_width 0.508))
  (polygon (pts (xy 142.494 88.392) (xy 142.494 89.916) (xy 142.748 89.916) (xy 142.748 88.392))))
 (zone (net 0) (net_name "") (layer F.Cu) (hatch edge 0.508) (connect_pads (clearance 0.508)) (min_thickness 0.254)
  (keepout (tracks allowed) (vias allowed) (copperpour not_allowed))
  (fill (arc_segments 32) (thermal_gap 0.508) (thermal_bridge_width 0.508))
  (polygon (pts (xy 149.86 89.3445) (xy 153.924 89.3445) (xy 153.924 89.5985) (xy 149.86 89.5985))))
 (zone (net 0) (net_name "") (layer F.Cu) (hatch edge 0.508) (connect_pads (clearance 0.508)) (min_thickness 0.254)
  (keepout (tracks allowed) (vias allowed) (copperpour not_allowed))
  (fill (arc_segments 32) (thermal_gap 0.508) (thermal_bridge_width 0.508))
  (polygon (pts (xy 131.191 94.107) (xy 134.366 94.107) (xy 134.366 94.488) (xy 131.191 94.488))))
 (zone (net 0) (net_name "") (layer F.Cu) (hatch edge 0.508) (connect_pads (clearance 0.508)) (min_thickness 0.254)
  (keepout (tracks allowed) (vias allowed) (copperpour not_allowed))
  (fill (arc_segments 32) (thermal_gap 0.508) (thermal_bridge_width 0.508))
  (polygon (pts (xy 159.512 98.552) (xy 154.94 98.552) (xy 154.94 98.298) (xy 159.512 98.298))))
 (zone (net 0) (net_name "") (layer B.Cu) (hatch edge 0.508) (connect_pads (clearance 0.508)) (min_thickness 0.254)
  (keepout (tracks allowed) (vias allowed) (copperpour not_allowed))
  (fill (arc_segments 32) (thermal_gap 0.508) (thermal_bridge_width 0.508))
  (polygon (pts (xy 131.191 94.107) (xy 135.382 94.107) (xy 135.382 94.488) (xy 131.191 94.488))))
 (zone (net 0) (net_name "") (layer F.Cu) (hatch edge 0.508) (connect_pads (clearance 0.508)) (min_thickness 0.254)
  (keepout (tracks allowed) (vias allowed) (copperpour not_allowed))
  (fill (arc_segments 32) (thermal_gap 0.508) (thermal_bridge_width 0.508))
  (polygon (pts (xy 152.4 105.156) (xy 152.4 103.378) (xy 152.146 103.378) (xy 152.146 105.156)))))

